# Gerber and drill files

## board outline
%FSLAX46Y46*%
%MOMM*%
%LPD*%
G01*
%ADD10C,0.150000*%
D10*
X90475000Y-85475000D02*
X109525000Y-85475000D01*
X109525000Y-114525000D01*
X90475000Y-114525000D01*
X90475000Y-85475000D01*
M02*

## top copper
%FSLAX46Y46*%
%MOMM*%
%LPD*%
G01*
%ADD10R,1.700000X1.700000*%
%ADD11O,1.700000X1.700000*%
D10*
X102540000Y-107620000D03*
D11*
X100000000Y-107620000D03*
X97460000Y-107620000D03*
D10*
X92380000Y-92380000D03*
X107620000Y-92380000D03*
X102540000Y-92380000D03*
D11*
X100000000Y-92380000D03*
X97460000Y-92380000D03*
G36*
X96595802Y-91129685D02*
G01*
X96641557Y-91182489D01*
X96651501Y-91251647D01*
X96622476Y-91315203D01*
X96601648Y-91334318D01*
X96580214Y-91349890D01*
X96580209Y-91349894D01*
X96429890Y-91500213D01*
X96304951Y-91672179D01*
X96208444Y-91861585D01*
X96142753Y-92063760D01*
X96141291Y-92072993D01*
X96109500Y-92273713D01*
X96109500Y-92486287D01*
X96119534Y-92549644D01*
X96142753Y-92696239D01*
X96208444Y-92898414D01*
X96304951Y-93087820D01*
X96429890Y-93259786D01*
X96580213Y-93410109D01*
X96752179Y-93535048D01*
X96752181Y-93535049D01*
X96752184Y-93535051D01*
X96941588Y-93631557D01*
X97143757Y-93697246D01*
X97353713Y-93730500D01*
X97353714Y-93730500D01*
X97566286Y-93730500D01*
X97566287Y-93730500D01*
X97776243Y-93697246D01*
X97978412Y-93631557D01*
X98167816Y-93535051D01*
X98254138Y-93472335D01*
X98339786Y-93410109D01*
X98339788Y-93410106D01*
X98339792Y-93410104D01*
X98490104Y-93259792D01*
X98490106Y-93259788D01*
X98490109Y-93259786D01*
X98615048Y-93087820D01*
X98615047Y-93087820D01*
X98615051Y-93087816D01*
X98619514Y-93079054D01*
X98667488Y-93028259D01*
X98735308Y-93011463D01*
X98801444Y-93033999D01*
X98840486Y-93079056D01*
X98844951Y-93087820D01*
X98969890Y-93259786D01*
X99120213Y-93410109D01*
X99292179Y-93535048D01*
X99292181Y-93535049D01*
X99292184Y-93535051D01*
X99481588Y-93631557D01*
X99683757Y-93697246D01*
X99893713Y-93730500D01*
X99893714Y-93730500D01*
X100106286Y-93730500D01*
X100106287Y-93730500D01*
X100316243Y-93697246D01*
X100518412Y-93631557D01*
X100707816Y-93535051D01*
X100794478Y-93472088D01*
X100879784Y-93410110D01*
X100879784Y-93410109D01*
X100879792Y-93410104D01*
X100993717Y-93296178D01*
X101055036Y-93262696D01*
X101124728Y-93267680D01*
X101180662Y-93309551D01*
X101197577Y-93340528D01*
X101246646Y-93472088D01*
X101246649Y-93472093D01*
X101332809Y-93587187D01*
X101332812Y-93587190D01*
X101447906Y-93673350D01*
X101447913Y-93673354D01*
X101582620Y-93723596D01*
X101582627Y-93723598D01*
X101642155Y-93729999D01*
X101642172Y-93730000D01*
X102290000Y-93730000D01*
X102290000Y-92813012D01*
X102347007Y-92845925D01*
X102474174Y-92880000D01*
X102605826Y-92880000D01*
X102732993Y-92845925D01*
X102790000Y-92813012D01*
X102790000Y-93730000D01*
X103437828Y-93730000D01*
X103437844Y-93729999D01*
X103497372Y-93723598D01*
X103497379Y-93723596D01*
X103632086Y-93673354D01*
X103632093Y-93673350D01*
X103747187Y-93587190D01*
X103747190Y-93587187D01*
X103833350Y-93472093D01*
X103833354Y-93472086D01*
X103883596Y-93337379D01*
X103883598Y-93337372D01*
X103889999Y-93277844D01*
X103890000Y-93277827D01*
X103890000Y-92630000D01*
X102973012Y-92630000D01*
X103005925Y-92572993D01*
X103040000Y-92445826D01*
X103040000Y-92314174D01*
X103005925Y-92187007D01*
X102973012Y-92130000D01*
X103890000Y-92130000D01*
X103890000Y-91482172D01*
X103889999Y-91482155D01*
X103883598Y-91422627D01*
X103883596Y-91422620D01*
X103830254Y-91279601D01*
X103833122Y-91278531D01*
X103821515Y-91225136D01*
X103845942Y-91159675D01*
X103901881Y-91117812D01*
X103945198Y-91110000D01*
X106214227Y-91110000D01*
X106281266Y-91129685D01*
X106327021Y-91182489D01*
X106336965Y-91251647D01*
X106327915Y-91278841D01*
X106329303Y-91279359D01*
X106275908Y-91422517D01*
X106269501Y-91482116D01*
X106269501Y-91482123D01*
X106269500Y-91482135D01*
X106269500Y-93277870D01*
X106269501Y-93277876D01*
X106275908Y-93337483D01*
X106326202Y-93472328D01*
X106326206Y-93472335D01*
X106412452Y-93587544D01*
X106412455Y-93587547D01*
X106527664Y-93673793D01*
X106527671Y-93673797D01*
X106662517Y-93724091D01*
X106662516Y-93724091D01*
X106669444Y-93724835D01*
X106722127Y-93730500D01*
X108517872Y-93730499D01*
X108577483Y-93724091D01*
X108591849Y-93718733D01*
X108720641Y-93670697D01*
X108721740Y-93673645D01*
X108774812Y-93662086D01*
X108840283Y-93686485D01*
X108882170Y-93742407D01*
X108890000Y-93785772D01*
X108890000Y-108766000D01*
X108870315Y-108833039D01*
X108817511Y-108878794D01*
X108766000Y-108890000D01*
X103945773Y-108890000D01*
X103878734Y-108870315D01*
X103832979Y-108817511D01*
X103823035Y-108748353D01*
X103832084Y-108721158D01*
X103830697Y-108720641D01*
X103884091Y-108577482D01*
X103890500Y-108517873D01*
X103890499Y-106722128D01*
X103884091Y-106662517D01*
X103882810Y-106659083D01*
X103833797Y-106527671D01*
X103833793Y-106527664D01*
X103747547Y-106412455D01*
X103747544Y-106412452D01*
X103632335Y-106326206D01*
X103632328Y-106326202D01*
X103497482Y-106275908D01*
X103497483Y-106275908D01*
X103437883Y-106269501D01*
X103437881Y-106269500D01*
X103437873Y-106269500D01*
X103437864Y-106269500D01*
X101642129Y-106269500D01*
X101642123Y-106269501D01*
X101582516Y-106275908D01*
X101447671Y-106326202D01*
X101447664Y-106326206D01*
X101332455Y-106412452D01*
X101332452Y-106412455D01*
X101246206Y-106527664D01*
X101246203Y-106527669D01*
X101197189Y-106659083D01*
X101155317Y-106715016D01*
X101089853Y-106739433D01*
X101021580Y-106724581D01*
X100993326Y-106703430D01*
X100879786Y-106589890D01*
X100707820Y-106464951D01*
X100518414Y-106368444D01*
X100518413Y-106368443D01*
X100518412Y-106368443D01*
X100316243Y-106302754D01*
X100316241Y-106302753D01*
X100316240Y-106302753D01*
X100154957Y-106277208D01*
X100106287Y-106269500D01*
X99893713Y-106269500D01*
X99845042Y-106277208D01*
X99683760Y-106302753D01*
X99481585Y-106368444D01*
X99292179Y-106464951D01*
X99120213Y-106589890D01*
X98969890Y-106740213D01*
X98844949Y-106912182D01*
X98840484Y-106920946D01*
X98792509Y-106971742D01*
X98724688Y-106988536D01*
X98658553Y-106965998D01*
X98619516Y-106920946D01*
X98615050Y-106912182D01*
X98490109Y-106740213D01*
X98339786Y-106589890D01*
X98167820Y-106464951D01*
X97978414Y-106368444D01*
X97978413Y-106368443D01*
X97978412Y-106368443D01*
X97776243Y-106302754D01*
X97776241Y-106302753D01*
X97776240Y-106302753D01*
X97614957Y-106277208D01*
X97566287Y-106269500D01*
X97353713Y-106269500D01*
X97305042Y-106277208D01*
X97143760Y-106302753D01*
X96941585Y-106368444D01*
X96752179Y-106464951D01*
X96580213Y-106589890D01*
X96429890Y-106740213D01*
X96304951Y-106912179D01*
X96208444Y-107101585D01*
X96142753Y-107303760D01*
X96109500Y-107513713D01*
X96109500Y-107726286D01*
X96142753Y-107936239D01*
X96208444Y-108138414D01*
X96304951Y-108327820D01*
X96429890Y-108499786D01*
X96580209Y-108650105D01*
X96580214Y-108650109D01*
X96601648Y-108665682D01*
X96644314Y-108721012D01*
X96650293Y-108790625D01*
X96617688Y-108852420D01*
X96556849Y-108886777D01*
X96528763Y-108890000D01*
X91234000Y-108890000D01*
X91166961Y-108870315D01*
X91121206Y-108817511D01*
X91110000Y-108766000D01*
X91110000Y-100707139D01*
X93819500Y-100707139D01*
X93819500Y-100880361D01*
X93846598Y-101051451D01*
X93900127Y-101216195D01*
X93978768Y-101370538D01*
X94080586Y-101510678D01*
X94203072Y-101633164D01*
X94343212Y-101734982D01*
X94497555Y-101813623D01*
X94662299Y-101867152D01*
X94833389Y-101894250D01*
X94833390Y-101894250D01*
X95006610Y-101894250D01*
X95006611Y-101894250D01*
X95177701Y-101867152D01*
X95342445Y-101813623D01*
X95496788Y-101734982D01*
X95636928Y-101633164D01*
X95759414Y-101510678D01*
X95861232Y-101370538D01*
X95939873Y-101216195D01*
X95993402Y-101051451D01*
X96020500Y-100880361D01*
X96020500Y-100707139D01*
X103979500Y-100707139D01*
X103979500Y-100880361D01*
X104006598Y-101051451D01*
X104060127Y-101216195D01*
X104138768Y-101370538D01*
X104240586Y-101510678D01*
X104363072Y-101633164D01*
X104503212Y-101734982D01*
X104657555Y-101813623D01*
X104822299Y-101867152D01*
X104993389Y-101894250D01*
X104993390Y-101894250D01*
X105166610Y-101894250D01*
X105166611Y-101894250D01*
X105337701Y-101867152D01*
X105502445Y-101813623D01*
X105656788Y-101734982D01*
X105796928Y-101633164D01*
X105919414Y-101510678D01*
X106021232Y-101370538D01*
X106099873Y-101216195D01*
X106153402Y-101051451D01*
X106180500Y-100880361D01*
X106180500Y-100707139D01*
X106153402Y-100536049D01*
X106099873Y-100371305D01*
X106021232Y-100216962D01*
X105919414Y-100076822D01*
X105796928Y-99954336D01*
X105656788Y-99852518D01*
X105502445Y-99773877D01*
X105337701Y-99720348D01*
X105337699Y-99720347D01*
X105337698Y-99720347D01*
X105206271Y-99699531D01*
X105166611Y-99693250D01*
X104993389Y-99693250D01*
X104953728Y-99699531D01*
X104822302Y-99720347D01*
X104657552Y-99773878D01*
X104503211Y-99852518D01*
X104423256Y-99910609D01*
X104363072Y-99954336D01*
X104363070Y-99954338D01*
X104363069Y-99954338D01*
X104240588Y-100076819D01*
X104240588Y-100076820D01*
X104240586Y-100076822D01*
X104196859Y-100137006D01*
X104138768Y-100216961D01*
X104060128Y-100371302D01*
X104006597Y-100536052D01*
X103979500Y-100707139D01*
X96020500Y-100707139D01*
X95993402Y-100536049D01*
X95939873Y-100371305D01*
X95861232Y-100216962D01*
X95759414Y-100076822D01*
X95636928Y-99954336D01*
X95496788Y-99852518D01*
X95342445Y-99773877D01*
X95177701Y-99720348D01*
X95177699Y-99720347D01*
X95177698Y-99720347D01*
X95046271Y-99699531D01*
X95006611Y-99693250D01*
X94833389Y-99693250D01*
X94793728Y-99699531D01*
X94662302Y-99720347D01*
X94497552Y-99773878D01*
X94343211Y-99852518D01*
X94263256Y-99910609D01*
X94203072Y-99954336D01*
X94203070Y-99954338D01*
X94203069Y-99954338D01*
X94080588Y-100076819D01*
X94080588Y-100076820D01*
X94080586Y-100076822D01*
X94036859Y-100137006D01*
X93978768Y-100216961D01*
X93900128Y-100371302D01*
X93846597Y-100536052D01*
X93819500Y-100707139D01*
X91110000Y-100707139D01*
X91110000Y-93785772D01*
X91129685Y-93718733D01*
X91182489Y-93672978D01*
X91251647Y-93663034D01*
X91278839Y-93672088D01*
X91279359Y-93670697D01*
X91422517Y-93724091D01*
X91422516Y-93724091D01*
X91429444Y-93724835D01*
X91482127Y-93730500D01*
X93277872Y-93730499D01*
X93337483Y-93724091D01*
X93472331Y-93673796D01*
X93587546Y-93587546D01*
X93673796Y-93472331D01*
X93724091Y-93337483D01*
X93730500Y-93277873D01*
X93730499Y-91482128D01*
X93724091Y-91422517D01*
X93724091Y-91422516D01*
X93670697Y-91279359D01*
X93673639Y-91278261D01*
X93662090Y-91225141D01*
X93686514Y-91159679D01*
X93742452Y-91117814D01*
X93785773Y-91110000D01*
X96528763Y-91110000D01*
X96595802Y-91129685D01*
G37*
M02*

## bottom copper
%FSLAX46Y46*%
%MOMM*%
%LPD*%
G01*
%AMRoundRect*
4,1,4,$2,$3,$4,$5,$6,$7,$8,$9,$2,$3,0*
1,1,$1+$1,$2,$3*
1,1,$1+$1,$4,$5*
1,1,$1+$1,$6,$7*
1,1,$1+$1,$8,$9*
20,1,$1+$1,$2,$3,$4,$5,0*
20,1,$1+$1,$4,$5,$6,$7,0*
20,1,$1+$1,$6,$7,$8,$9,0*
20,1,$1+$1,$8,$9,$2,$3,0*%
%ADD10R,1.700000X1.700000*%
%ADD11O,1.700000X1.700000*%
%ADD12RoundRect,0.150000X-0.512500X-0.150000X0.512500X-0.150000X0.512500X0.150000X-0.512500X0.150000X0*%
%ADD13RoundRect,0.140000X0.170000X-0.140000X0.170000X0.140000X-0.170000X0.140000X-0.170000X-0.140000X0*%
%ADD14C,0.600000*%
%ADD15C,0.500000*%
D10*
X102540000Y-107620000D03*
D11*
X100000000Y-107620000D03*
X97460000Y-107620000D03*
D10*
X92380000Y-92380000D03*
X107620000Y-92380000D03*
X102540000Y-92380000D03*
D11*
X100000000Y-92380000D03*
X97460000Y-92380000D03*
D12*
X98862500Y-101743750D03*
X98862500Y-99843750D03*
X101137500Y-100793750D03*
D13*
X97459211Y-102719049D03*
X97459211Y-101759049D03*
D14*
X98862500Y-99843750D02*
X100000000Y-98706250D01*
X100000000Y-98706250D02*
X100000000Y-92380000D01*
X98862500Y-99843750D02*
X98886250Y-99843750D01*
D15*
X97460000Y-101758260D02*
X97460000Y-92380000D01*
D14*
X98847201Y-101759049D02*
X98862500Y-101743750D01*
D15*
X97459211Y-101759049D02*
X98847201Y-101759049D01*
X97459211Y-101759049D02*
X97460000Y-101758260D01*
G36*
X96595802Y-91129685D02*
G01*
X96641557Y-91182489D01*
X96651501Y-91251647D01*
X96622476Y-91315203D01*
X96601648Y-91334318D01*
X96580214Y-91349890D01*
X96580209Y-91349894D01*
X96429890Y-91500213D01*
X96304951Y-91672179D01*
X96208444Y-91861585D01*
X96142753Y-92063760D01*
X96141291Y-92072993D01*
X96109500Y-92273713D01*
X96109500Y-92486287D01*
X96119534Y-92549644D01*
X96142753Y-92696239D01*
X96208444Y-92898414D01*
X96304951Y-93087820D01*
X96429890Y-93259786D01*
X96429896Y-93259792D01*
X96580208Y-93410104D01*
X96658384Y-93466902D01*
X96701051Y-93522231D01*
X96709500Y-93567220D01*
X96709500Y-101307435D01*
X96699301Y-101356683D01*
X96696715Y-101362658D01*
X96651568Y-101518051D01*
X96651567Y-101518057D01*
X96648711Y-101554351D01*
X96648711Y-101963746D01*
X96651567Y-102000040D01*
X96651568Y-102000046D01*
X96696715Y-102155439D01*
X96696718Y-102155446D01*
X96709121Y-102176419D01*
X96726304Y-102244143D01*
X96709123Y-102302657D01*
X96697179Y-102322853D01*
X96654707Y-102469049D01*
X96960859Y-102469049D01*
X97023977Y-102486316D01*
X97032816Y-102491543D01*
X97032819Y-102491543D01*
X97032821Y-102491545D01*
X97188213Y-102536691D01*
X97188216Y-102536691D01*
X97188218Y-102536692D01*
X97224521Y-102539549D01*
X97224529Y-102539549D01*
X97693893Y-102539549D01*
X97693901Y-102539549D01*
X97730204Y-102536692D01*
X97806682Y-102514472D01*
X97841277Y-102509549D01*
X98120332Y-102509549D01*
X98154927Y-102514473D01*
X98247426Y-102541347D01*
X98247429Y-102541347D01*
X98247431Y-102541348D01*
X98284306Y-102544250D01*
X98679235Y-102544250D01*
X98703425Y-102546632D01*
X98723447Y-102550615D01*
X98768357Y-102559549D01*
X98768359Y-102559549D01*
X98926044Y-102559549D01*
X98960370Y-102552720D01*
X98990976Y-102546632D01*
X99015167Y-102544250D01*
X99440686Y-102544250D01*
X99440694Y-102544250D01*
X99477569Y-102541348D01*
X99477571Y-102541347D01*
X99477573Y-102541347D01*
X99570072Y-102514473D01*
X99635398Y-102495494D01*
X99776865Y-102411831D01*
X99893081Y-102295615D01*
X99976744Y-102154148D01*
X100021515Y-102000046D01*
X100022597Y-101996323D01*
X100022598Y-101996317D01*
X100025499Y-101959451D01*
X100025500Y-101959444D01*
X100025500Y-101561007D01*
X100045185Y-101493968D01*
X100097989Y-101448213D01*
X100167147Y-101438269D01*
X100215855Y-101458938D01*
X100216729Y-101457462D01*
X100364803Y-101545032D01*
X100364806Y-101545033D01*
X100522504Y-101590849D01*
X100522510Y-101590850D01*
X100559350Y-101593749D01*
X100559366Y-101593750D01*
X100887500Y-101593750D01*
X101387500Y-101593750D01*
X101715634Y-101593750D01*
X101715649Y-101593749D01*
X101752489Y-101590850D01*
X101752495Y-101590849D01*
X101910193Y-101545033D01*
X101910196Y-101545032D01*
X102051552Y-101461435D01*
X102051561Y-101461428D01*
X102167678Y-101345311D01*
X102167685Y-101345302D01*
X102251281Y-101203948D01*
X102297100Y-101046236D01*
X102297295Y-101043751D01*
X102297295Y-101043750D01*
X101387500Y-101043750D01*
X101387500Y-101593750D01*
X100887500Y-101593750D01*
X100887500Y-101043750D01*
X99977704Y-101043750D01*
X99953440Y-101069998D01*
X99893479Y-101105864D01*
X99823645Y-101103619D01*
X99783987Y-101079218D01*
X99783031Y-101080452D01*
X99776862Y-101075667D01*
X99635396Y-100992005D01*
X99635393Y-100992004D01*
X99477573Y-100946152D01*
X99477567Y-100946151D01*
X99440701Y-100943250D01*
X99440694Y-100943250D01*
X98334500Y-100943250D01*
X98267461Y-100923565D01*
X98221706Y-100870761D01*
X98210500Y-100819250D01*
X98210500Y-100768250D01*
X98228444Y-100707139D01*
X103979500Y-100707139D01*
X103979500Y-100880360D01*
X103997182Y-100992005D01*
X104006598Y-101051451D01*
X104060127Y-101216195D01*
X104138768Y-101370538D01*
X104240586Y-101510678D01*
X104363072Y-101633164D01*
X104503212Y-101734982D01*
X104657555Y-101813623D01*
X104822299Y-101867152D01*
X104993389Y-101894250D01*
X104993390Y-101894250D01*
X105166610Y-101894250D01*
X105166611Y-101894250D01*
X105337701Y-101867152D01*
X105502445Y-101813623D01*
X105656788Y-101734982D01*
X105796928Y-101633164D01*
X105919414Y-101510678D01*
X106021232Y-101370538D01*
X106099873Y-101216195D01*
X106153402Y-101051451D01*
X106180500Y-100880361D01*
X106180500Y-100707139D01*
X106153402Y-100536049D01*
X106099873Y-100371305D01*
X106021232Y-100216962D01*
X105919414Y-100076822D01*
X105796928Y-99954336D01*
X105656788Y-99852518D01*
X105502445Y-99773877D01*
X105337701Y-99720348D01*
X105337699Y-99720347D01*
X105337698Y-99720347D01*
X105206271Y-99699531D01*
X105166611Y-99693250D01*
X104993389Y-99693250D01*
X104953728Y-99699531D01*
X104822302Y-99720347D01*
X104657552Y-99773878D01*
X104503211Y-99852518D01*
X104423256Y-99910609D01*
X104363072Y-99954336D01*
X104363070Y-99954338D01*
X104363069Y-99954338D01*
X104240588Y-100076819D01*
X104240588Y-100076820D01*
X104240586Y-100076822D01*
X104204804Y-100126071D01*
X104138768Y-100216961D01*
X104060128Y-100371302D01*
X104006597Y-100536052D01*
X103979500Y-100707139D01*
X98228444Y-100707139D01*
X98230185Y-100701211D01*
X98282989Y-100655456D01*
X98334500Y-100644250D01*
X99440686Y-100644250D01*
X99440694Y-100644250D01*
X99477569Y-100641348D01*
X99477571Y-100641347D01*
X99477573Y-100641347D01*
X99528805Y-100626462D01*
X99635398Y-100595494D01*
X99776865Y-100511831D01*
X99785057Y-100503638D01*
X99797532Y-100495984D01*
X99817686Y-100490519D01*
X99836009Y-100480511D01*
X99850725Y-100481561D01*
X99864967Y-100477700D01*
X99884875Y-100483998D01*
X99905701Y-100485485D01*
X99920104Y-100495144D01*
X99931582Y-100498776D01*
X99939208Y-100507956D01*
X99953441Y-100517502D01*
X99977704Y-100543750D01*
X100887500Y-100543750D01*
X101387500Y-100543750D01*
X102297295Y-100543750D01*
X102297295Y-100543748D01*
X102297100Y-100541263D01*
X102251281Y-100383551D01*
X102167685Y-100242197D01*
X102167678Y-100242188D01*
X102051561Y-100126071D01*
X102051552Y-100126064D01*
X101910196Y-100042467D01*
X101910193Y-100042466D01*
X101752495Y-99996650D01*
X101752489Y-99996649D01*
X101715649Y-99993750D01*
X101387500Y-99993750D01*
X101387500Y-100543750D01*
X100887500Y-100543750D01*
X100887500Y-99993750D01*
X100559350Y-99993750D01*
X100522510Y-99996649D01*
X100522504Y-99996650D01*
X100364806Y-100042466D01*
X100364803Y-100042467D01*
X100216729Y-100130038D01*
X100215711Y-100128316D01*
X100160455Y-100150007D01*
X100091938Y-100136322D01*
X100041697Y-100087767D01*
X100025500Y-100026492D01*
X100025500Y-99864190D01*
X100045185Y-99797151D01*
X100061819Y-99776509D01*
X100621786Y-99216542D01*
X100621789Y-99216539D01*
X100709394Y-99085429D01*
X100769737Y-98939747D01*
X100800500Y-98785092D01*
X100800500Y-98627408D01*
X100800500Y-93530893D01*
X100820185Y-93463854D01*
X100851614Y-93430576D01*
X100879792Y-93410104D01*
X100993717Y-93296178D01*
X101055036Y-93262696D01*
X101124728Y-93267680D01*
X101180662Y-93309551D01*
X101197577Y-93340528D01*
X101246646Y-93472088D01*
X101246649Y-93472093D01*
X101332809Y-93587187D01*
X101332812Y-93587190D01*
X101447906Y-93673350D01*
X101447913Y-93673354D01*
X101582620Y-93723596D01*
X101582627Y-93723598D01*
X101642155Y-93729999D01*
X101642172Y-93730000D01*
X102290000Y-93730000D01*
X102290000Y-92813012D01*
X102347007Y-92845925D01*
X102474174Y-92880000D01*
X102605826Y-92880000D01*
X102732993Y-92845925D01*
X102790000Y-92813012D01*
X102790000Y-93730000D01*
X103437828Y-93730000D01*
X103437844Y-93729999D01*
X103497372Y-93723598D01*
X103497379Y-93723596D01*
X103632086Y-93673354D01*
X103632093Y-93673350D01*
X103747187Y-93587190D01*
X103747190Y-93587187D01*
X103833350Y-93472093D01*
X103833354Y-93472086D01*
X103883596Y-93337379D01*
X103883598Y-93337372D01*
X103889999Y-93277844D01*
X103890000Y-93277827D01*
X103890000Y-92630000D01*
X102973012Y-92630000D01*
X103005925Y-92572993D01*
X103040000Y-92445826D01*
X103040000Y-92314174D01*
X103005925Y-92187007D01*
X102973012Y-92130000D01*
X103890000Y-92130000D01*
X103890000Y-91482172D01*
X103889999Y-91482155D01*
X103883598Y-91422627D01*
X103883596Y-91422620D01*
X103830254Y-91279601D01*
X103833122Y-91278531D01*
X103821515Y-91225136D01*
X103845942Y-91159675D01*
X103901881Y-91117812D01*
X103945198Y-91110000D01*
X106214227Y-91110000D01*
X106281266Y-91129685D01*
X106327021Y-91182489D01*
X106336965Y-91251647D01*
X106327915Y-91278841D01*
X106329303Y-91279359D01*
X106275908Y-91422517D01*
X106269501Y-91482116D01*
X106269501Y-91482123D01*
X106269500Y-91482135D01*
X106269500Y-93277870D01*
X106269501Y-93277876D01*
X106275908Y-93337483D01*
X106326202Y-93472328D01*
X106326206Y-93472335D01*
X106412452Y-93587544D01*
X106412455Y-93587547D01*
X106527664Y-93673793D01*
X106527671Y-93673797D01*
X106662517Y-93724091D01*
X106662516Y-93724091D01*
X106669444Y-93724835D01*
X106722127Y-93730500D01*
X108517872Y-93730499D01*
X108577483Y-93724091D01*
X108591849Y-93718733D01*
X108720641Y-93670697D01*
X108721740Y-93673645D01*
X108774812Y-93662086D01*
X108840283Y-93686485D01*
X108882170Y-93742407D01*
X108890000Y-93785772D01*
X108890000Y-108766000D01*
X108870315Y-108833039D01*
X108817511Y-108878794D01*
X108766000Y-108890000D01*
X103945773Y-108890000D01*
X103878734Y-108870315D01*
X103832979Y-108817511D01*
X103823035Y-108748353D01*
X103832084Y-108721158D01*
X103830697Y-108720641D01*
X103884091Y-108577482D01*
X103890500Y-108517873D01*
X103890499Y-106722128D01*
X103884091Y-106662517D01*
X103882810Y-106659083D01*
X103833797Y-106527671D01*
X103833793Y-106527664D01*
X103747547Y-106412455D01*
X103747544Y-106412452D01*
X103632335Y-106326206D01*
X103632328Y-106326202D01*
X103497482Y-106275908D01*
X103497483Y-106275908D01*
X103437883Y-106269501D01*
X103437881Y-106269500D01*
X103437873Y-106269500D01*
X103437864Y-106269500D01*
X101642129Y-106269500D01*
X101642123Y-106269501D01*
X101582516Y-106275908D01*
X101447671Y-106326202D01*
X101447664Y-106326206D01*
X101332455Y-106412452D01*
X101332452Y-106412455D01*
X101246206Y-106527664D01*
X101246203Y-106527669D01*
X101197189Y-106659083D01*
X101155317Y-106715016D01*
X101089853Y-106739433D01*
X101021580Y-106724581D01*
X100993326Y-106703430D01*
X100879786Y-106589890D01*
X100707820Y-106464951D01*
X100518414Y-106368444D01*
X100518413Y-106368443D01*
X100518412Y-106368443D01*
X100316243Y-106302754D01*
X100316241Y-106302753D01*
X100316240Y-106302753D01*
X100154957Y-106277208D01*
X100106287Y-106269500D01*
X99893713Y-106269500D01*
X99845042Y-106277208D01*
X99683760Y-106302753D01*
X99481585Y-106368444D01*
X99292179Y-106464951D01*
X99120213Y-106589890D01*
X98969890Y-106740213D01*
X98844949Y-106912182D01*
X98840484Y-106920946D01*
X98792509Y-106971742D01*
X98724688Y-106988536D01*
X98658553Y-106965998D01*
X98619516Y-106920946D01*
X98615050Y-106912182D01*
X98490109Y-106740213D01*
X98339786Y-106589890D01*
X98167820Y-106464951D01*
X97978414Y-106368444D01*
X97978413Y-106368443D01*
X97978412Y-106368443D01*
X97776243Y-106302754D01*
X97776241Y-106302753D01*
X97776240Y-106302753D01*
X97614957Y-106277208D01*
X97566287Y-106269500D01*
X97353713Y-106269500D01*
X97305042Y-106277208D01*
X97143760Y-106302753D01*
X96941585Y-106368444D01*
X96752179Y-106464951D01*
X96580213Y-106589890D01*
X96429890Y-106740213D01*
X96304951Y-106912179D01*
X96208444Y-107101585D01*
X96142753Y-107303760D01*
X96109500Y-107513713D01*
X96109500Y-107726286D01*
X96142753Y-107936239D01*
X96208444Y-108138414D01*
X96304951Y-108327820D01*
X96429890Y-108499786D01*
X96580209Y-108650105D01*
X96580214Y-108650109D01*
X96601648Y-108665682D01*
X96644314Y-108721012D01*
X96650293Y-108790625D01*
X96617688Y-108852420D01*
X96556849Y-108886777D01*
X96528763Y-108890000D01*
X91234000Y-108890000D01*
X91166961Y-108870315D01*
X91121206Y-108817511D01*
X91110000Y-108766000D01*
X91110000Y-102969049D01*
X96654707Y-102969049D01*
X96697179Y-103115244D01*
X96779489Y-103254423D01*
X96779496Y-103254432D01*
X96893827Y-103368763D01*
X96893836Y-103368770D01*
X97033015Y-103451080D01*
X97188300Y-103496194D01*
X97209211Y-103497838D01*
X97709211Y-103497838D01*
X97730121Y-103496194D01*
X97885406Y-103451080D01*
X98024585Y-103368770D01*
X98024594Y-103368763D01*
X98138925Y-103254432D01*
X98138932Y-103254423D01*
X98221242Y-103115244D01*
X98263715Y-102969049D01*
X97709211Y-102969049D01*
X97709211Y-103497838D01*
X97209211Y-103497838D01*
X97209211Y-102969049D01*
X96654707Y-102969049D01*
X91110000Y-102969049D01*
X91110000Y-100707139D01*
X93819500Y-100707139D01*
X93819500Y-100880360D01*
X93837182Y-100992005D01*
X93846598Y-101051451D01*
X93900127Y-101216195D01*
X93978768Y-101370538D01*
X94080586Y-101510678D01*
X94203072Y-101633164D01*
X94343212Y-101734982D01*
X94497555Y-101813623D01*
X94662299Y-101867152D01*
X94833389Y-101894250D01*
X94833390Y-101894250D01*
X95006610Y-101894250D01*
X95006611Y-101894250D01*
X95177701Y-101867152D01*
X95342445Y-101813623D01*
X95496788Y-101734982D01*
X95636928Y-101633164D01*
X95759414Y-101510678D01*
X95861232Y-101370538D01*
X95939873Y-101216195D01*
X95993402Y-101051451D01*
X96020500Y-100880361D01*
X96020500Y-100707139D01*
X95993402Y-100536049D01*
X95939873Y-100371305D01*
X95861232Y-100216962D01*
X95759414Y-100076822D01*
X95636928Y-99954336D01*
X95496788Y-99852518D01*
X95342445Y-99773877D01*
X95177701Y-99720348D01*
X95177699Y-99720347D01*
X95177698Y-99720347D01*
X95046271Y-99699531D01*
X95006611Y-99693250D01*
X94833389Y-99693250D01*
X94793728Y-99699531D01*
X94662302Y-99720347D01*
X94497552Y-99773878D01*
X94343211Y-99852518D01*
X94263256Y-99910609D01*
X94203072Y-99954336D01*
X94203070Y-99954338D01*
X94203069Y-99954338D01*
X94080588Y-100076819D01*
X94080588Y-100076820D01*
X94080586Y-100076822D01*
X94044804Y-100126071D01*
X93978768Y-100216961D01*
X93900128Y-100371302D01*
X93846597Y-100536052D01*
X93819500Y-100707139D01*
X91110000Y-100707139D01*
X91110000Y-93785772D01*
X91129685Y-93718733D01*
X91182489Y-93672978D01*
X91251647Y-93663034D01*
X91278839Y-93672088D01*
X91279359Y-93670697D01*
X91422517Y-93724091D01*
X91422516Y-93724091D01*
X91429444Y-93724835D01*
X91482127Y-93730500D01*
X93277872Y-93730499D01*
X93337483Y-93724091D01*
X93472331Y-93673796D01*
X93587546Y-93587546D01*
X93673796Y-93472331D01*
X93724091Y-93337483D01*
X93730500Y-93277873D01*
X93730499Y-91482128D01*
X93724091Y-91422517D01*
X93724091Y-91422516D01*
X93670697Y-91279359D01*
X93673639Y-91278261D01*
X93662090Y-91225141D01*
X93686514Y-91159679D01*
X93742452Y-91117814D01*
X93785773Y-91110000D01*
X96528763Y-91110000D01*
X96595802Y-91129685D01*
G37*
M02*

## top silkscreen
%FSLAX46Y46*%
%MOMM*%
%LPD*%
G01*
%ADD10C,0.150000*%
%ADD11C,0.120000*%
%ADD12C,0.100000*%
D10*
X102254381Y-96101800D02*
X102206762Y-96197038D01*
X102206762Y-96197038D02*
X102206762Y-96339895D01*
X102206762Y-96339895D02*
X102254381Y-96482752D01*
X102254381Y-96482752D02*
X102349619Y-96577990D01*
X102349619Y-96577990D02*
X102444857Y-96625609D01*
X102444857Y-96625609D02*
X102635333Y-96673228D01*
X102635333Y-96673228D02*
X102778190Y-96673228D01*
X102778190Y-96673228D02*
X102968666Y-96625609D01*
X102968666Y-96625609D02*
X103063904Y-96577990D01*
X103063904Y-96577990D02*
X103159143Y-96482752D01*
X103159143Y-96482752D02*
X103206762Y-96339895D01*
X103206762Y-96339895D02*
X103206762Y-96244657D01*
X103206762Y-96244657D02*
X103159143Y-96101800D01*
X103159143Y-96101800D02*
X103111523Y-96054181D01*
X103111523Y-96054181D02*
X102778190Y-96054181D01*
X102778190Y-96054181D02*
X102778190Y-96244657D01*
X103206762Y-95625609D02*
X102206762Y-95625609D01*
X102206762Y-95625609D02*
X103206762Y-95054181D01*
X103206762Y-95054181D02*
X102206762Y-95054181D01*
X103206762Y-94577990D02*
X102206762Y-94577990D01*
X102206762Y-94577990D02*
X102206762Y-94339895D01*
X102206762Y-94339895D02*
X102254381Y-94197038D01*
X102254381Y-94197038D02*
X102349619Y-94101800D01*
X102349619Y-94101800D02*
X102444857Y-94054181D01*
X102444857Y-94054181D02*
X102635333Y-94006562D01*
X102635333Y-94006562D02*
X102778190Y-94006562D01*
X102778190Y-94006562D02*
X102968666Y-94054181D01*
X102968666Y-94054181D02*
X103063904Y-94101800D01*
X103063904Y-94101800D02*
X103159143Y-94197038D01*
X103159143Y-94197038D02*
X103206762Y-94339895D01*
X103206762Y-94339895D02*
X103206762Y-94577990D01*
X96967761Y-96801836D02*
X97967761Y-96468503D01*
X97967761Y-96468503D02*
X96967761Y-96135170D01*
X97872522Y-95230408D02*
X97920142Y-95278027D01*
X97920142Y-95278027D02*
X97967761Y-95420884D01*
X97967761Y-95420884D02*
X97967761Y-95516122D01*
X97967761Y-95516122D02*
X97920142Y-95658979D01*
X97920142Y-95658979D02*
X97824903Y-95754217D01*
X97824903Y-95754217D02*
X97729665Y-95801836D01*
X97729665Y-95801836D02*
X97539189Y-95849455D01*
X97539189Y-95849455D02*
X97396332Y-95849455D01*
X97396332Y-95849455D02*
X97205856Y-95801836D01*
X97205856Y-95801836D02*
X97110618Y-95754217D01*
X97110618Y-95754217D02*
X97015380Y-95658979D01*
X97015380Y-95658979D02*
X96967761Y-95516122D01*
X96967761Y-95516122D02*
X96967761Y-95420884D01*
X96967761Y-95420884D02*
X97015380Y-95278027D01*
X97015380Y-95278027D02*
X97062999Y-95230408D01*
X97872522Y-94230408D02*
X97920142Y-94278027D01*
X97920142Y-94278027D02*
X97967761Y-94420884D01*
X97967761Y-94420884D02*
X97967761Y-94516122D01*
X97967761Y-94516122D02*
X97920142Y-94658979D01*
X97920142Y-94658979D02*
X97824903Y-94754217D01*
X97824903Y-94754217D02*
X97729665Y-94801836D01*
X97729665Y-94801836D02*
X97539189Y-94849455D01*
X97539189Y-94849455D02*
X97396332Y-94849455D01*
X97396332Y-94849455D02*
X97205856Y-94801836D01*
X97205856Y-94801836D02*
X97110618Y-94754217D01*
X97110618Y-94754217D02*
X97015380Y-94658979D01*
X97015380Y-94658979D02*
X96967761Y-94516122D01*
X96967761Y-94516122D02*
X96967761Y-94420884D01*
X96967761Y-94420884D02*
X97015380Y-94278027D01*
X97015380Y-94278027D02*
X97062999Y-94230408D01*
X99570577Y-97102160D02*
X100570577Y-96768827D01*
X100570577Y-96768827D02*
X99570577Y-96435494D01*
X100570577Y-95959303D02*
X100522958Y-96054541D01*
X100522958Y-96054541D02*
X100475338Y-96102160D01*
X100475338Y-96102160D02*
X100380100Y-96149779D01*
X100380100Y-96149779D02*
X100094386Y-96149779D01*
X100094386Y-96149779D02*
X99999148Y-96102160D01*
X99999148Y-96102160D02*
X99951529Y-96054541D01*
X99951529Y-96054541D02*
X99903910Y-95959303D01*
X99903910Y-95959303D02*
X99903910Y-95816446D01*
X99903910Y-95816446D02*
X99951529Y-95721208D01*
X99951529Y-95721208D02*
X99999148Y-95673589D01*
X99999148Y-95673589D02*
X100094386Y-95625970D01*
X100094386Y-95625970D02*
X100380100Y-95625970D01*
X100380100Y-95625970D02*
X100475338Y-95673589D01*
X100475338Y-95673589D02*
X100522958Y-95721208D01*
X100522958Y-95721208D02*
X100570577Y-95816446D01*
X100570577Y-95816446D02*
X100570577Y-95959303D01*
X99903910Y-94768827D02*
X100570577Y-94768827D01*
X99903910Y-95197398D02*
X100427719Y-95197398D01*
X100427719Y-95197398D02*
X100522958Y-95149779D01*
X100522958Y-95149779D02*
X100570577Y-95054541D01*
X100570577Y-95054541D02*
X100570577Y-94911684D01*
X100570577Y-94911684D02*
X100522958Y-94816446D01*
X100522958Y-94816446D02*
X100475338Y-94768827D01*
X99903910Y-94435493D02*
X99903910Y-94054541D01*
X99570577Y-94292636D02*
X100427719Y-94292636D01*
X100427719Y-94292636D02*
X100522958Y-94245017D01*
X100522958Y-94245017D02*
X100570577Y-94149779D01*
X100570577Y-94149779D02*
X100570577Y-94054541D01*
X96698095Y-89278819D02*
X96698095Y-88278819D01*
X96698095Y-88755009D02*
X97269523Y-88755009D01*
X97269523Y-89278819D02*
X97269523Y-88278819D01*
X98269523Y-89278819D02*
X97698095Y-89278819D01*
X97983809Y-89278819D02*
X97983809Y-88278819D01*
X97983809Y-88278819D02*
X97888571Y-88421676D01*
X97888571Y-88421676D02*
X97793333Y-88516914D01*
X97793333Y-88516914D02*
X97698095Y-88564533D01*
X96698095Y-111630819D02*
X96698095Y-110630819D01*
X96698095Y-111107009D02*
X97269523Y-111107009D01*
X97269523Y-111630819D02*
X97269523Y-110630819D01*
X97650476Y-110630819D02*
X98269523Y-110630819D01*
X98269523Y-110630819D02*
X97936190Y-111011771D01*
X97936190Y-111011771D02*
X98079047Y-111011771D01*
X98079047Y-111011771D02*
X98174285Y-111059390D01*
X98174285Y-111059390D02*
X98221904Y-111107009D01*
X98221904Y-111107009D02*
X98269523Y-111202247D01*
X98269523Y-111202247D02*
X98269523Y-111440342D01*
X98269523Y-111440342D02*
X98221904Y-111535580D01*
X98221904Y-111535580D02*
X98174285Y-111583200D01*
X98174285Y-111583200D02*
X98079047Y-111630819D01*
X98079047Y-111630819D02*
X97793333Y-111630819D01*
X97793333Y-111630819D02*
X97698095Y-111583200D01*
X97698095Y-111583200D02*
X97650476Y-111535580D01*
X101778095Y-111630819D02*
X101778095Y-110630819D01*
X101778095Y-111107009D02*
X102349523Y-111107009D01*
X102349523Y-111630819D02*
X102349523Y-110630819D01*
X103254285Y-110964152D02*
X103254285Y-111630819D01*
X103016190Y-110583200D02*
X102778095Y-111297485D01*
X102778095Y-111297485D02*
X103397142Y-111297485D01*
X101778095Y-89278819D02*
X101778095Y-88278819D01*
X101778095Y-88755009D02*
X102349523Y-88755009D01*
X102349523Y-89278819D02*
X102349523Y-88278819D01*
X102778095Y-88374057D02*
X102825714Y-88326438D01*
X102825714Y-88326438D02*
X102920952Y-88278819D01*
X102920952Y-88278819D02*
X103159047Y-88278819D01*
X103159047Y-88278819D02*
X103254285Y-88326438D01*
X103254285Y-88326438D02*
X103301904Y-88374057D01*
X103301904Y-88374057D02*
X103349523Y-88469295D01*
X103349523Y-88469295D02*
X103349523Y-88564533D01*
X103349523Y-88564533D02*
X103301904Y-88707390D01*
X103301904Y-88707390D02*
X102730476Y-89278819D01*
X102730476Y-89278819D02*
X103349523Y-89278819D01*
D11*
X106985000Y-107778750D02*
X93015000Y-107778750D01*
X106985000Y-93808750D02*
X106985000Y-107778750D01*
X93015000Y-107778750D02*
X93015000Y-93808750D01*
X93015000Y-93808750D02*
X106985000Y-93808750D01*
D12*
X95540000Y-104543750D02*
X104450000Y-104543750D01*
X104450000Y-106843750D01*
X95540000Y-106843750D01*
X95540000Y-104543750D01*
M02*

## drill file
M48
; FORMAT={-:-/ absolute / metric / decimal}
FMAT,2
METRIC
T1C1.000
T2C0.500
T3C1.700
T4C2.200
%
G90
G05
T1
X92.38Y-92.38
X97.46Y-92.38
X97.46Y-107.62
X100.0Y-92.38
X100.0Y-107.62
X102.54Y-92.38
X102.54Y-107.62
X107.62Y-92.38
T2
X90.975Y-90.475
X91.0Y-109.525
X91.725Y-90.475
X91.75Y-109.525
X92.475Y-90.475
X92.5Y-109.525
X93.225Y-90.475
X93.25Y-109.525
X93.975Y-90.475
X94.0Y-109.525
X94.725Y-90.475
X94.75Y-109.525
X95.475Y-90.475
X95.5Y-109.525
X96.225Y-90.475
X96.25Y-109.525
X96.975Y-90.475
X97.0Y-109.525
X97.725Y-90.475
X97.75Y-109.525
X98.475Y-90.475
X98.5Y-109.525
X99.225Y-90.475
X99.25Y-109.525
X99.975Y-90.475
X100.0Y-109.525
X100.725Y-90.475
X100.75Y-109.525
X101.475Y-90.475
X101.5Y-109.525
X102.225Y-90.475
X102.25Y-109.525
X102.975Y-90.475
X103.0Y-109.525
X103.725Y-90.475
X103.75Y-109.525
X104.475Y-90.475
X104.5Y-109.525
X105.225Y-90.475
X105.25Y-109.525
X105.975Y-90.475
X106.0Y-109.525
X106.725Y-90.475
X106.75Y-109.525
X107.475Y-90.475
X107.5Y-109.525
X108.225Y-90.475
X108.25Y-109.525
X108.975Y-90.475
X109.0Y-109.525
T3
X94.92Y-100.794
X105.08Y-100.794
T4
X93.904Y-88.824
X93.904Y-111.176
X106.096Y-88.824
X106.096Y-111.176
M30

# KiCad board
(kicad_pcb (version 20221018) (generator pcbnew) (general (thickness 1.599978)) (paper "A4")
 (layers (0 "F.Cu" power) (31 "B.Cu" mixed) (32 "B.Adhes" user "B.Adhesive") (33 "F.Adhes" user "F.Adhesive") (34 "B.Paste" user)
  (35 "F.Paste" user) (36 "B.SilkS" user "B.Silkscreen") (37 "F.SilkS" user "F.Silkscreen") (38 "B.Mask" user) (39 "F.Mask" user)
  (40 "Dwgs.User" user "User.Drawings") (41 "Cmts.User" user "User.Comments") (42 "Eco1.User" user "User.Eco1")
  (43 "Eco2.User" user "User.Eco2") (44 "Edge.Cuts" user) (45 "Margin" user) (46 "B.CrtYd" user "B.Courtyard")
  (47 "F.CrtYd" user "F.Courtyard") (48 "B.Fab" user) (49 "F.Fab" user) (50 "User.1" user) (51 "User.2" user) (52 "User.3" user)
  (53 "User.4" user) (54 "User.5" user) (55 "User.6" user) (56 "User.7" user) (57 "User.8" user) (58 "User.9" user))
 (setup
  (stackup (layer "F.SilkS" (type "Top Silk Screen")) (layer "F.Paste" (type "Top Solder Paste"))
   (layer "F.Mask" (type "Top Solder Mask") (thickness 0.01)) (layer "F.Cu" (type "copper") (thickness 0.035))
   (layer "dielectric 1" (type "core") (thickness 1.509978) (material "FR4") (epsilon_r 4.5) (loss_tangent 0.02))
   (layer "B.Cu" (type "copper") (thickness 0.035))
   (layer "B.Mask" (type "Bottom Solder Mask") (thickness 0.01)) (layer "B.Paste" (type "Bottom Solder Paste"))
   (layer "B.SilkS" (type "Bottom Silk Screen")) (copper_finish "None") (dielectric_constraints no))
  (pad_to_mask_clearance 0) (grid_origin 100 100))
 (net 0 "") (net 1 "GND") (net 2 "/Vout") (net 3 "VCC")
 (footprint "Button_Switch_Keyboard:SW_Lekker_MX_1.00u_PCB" (layer "F.Cu") (at 100 100.79375 180)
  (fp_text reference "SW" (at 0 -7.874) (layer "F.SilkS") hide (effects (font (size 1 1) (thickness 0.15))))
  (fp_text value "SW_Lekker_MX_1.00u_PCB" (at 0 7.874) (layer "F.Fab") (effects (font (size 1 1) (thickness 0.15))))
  (fp_line (start -6.985 -6.985) (end 6.985 -6.985) (stroke (width 0.12) (type solid)) (layer "F.SilkS"))
  (fp_line (start -6.985 6.985) (end -6.985 -6.985) (stroke (width 0.12) (type solid)) (layer "F.SilkS"))
  (fp_line (start 6.985 -6.985) (end 6.985 6.985) (stroke (width 0.12) (type solid)) (layer "F.SilkS"))
  (fp_line (start 6.985 6.985) (end -6.985 6.985) (stroke (width 0.12) (type solid)) (layer "F.SilkS"))
  (fp_rect (start -4.45 -6.05) (end 4.46 -3.75) (stroke (width 0.1) (type default)) (fill none) (layer "F.SilkS"))
  (pad "" np_thru_hole circle (at -5.08 0 180) (size 1.7 1.7) (drill 1.7) (layers "*.Cu" "*.Mask"))
  (pad "" np_thru_hole circle (at 5.08 0 180) (size 1.7 1.7) (drill 1.7) (layers "*.Cu" "*.Mask")))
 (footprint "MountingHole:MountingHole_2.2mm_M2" (layer "F.Cu") (at 93.904 88.824)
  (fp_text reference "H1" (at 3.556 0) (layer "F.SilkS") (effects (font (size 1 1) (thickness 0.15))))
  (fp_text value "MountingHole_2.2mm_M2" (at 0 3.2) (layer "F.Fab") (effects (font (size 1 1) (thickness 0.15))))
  (pad "" np_thru_hole circle (at 0 0) (size 2.2 2.2) (drill 2.2) (layers "*.Cu" "*.Mask")))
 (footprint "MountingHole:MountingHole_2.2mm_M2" (layer "F.Cu") (at 93.904 111.176)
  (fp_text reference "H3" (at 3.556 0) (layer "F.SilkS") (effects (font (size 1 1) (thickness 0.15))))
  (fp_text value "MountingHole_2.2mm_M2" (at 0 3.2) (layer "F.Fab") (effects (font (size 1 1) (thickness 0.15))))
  (pad "" np_thru_hole circle (at 0 0) (size 2.2 2.2) (drill 2.2) (layers "*.Cu" "*.Mask")))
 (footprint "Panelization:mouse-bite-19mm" (layer "F.Cu") (at 100 109.525)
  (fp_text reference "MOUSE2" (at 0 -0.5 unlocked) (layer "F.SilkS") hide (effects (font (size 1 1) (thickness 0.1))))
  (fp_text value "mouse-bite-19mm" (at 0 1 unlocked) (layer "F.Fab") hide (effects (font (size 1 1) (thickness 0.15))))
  (pad "" np_thru_hole circle (at -9 0) (size 0.5 0.5) (drill 0.5) (layers "*.Cu" "*.Mask"))
  (pad "" np_thru_hole circle (at -8.25 0) (size 0.5 0.5) (drill 0.5) (layers "*.Cu" "*.Mask"))
  (pad "" np_thru_hole circle (at -7.5 0) (size 0.5 0.5) (drill 0.5) (layers "*.Cu" "*.Mask"))
  (pad "" np_thru_hole circle (at -6.75 0) (size 0.5 0.5) (drill 0.5) (layers "*.Cu" "*.Mask"))
  (pad "" np_thru_hole circle (at -6 0) (size 0.5 0.5) (drill 0.5) (layers "*.Cu" "*.Mask"))
  (pad "" np_thru_hole circle (at -5.25 0) (size 0.5 0.5) (drill 0.5) (layers "*.Cu" "*.Mask"))
  (pad "" np_thru_hole circle (at -4.5 0) (size 0.5 0.5) (drill 0.5) (layers "*.Cu" "*.Mask"))
  (pad "" np_thru_hole circle (at -3.75 0) (size 0.5 0.5) (drill 0.5) (layers "*.Cu" "*.Mask"))
  (pad "" np_thru_hole circle (at -3 0) (size 0.5 0.5) (drill 0.5) (layers "*.Cu" "*.Mask"))
  (pad "" np_thru_hole circle (at -2.25 0) (size 0.5 0.5) (drill 0.5) (layers "*.Cu" "*.Mask"))
  (pad "" np_thru_hole circle (at -1.5 0) (size 0.5 0.5) (drill 0.5) (layers "*.Cu" "*.Mask"))
  (pad "" np_thru_hole circle (at -0.75 0) (size 0.5 0.5) (drill 0.5) (layers "*.Cu" "*.Mask"))
  (pad "" np_thru_hole circle (at 0 0) (size 0.5 0.5) (drill 0.5) (layers "*.Cu" "*.Mask"))
  (pad "" np_thru_hole circle (at 0.75 0) (size 0.5 0.5) (drill 0.5) (layers "*.Cu" "*.Mask"))
  (pad "" np_thru_hole circle (at 1.5 0) (size 0.5 0.5) (drill 0.5) (layers "*.Cu" "*.Mask"))
  (pad "" np_thru_hole circle (at 2.25 0) (size 0.5 0.5) (drill 0.5) (layers "*.Cu" "*.Mask"))
  (pad "" np_thru_hole circle (at 3 0) (size 0.5 0.5) (drill 0.5) (layers "*.Cu" "*.Mask"))
  (pad "" np_thru_hole circle (at 3.75 0) (size 0.5 0.5) (drill 0.5) (layers "*.Cu" "*.Mask"))
  (pad "" np_thru_hole circle (at 4.5 0) (size 0.5 0.5) (drill 0.5) (layers "*.Cu" "*.Mask"))
  (pad "" np_thru_hole circle (at 5.25 0) (size 0.5 0.5) (drill 0.5) (layers "*.Cu" "*.Mask"))
  (pad "" np_thru_hole circle (at 6 0) (size 0.5 0.5) (drill 0.5) (layers "*.Cu" "*.Mask"))
  (pad "" np_thru_hole circle (at 6.75 0) (size 0.5 0.5) (drill 0.5) (layers "*.Cu" "*.Mask"))
  (pad "" np_thru_hole circle (at 7.5 0) (size 0.5 0.5) (drill 0.5) (layers "*.Cu" "*.Mask"))
  (pad "" np_thru_hole circle (at 8.25 0) (size 0.5 0.5) (drill 0.5) (layers "*.Cu" "*.Mask"))
  (pad "" np_thru_hole circle (at 9 0) (size 0.5 0.5) (drill 0.5) (layers "*.Cu" "*.Mask")))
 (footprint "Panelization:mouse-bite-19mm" (layer "F.Cu") (at 99.9746 90.475)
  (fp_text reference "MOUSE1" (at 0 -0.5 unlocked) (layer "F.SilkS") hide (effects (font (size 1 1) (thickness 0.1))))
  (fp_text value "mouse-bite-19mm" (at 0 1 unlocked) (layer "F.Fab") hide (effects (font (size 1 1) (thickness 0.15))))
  (pad "" np_thru_hole circle (at -9 0) (size 0.5 0.5) (drill 0.5) (layers "*.Cu" "*.Mask"))
  (pad "" np_thru_hole circle (at -8.25 0) (size 0.5 0.5) (drill 0.5) (layers "*.Cu" "*.Mask"))
  (pad "" np_thru_hole circle (at -7.5 0) (size 0.5 0.5) (drill 0.5) (layers "*.Cu" "*.Mask"))
  (pad "" np_thru_hole circle (at -6.75 0) (size 0.5 0.5) (drill 0.5) (layers "*.Cu" "*.Mask"))
  (pad "" np_thru_hole circle (at -6 0) (size 0.5 0.5) (drill 0.5) (layers "*.Cu" "*.Mask"))
  (pad "" np_thru_hole circle (at -5.25 0) (size 0.5 0.5) (drill 0.5) (layers "*.Cu" "*.Mask"))
  (pad "" np_thru_hole circle (at -4.5 0) (size 0.5 0.5) (drill 0.5) (layers "*.Cu" "*.Mask"))
  (pad "" np_thru_hole circle (at -3.75 0) (size 0.5 0.5) (drill 0.5) (layers "*.Cu" "*.Mask"))
  (pad "" np_thru_hole circle (at -3 0) (size 0.5 0.5) (drill 0.5) (layers "*.Cu" "*.Mask"))
  (pad "" np_thru_hole circle (at -2.25 0) (size 0.5 0.5) (drill 0.5) (layers "*.Cu" "*.Mask"))
  (pad "" np_thru_hole circle (at -1.5 0) (size 0.5 0.5) (drill 0.5) (layers "*.Cu" "*.Mask"))
  (pad "" np_thru_hole circle (at -0.75 0) (size 0.5 0.5) (drill 0.5) (layers "*.Cu" "*.Mask"))
  (pad "" np_thru_hole circle (at 0 0) (size 0.5 0.5) (drill 0.5) (layers "*.Cu" "*.Mask"))
  (pad "" np_thru_hole circle (at 0.75 0) (size 0.5 0.5) (drill 0.5) (layers "*.Cu" "*.Mask"))
  (pad "" np_thru_hole circle (at 1.5 0) (size 0.5 0.5) (drill 0.5) (layers "*.Cu" "*.Mask"))
  (pad "" np_thru_hole circle (at 2.25 0) (size 0.5 0.5) (drill 0.5) (layers "*.Cu" "*.Mask"))
  (pad "" np_thru_hole circle (at 3 0) (size 0.5 0.5) (drill 0.5) (layers "*.Cu" "*.Mask"))
  (pad "" np_thru_hole circle (at 3.75 0) (size 0.5 0.5) (drill 0.5) (layers "*.Cu" "*.Mask"))
  (pad "" np_thru_hole circle (at 4.5 0) (size 0.5 0.5) (drill 0.5) (layers "*.Cu" "*.Mask"))
  (pad "" np_thru_hole circle (at 5.25 0) (size 0.5 0.5) (drill 0.5) (layers "*.Cu" "*.Mask"))
  (pad "" np_thru_hole circle (at 6 0) (size 0.5 0.5) (drill 0.5) (layers "*.Cu" "*.Mask"))
  (pad "" np_thru_hole circle (at 6.75 0) (size 0.5 0.5) (drill 0.5) (layers "*.Cu" "*.Mask"))
  (pad "" np_thru_hole circle (at 7.5 0) (size 0.5 0.5) (drill 0.5) (layers "*.Cu" "*.Mask"))
  (pad "" np_thru_hole circle (at 8.25 0) (size 0.5 0.5) (drill 0.5) (layers "*.Cu" "*.Mask"))
  (pad "" np_thru_hole circle (at 9 0) (size 0.5 0.5) (drill 0.5) (layers "*.Cu" "*.Mask")))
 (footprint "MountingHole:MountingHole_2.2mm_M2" (layer "F.Cu") (at 106.096 111.176)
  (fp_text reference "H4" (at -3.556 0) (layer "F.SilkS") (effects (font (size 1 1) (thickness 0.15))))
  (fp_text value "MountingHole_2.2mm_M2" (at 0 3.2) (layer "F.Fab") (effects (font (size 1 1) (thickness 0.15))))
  (pad "" np_thru_hole circle (at 0 0) (size 2.2 2.2) (drill 2.2) (layers "*.Cu" "*.Mask")))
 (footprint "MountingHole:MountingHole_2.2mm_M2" (layer "F.Cu") (at 106.096 88.824)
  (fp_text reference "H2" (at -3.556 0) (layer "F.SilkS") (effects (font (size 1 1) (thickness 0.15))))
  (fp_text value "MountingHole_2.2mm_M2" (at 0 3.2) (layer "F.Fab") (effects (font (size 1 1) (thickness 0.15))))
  (pad "" np_thru_hole circle (at 0 0) (size 2.2 2.2) (drill 2.2) (layers "*.Cu" "*.Mask")))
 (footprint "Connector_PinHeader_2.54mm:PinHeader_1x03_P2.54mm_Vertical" (layer "B.Cu") (at 102.54 107.62 90)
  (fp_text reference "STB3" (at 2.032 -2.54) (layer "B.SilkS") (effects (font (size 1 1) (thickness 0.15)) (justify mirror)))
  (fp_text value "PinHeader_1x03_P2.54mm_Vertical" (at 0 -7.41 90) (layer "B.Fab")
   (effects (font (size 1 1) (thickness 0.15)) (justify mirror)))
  (pad "1" thru_hole rect (at 0 0 90) (size 1.7 1.7) (drill 1) (layers "*.Cu" "*.Mask"))
  (pad "2" thru_hole oval (at 0 -2.54 90) (size 1.7 1.7) (drill 1) (layers "*.Cu" "*.Mask"))
  (pad "3" thru_hole oval (at 0 -5.08 90) (size 1.7 1.7) (drill 1) (layers "*.Cu" "*.Mask")))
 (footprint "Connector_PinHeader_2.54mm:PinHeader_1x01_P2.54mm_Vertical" (layer "B.Cu") (at 92.38 92.38 180)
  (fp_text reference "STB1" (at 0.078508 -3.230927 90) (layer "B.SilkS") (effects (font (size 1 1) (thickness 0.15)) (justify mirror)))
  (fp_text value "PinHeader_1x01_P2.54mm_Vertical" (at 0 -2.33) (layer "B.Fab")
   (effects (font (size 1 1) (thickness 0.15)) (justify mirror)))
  (pad "1" thru_hole rect (at 0 0 180) (size 1.7 1.7) (drill 1) (layers "*.Cu" "*.Mask")))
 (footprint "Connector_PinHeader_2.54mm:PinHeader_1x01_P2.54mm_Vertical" (layer "B.Cu") (at 107.62 92.38 180)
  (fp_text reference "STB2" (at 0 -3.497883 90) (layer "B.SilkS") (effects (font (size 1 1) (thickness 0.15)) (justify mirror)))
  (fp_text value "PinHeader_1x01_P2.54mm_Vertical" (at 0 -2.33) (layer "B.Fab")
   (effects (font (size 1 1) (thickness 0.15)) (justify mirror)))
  (pad "1" thru_hole rect (at 0 0 180) (size 1.7 1.7) (drill 1) (layers "*.Cu" "*.Mask")))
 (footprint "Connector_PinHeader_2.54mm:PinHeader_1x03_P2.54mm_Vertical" (layer "B.Cu") (at 102.54 92.38 90)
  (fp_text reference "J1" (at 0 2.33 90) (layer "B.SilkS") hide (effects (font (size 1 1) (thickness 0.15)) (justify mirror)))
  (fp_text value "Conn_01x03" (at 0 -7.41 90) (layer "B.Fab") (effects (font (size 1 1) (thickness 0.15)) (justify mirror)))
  (pad "1" thru_hole rect (at 0 0 90) (size 1.7 1.7) (drill 1) (layers "*.Cu" "*.Mask") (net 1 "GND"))
  (pad "2" thru_hole oval (at 0 -2.54 90) (size 1.7 1.7) (drill 1) (layers "*.Cu" "*.Mask") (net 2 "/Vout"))
  (pad "3" thru_hole oval (at 0 -5.08 90) (size 1.7 1.7) (drill 1) (layers "*.Cu" "*.Mask") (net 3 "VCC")))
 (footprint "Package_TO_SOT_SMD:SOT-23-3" (layer "B.Cu") (at 100 100.79375)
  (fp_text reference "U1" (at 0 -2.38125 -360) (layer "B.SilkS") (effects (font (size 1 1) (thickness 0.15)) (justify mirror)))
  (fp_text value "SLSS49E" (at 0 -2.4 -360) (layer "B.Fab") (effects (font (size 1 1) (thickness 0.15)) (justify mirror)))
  (pad "1" smd roundrect (at -1.1375 0.95) (size 1.325 0.6) (layers "B.Cu" "B.Paste" "B.Mask") (roundrect_rratio 0.25) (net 3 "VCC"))
  (pad "2" smd roundrect (at -1.1375 -0.95) (size 1.325 0.6) (layers "B.Cu" "B.Paste" "B.Mask") (roundrect_rratio 0.25) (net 2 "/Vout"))
  (pad "3" smd roundrect (at 1.1375 0) (size 1.325 0.6) (layers "B.Cu" "B.Paste" "B.Mask") (roundrect_rratio 0.25) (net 1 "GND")))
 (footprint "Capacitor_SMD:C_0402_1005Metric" (layer "B.Cu") (at 97.459211 102.239049 90)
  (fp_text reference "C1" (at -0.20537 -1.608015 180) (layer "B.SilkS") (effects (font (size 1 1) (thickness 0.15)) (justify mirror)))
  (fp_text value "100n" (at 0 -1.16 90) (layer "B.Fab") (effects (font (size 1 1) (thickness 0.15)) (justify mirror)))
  (pad "1" smd roundrect (at -0.48 0 90) (size 0.56 0.62) (layers "B.Cu" "B.Paste" "B.Mask") (roundrect_rratio 0.25) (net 1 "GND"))
  (pad "2" smd roundrect (at 0.48 0 90) (size 0.56 0.62) (layers "B.Cu" "B.Paste" "B.Mask") (roundrect_rratio 0.25) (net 3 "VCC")))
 (gr_rect (start 90.475 85.475) (end 109.525 114.525) (stroke (width 0.15) (type default)) (fill none) (layer "Edge.Cuts"))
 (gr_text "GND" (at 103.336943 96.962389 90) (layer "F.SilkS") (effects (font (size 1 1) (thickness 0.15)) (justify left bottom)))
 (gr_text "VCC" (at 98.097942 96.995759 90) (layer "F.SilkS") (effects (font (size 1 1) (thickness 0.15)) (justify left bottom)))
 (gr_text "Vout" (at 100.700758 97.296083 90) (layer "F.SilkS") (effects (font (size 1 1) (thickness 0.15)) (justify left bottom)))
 (segment (start 98.8625 99.84375) (end 100 98.70625) (width 0.6) (layer "B.Cu") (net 2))
 (segment (start 100 98.70625) (end 100 92.38) (width 0.6) (layer "B.Cu") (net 2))
 (segment (start 98.8625 99.84375) (end 98.88625 99.84375) (width 0.6) (layer "B.Cu") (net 2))
 (segment (start 97.46 101.75826) (end 97.46 92.38) (width 0.5) (layer "B.Cu") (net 3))
 (segment (start 98.847201 101.759049) (end 98.8625 101.74375) (width 0.6) (layer "B.Cu") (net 3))
 (segment (start 97.459211 101.759049) (end 98.847201 101.759049) (width 0.5) (layer "B.Cu") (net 3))
 (segment (start 97.459211 101.759049) (end 97.46 101.75826) (width 0.5) (layer "B.Cu") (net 3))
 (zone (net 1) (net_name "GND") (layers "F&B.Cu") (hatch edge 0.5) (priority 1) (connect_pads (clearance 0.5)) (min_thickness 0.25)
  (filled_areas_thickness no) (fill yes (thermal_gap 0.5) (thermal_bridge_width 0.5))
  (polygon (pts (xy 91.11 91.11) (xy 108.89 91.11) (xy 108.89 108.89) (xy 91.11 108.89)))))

